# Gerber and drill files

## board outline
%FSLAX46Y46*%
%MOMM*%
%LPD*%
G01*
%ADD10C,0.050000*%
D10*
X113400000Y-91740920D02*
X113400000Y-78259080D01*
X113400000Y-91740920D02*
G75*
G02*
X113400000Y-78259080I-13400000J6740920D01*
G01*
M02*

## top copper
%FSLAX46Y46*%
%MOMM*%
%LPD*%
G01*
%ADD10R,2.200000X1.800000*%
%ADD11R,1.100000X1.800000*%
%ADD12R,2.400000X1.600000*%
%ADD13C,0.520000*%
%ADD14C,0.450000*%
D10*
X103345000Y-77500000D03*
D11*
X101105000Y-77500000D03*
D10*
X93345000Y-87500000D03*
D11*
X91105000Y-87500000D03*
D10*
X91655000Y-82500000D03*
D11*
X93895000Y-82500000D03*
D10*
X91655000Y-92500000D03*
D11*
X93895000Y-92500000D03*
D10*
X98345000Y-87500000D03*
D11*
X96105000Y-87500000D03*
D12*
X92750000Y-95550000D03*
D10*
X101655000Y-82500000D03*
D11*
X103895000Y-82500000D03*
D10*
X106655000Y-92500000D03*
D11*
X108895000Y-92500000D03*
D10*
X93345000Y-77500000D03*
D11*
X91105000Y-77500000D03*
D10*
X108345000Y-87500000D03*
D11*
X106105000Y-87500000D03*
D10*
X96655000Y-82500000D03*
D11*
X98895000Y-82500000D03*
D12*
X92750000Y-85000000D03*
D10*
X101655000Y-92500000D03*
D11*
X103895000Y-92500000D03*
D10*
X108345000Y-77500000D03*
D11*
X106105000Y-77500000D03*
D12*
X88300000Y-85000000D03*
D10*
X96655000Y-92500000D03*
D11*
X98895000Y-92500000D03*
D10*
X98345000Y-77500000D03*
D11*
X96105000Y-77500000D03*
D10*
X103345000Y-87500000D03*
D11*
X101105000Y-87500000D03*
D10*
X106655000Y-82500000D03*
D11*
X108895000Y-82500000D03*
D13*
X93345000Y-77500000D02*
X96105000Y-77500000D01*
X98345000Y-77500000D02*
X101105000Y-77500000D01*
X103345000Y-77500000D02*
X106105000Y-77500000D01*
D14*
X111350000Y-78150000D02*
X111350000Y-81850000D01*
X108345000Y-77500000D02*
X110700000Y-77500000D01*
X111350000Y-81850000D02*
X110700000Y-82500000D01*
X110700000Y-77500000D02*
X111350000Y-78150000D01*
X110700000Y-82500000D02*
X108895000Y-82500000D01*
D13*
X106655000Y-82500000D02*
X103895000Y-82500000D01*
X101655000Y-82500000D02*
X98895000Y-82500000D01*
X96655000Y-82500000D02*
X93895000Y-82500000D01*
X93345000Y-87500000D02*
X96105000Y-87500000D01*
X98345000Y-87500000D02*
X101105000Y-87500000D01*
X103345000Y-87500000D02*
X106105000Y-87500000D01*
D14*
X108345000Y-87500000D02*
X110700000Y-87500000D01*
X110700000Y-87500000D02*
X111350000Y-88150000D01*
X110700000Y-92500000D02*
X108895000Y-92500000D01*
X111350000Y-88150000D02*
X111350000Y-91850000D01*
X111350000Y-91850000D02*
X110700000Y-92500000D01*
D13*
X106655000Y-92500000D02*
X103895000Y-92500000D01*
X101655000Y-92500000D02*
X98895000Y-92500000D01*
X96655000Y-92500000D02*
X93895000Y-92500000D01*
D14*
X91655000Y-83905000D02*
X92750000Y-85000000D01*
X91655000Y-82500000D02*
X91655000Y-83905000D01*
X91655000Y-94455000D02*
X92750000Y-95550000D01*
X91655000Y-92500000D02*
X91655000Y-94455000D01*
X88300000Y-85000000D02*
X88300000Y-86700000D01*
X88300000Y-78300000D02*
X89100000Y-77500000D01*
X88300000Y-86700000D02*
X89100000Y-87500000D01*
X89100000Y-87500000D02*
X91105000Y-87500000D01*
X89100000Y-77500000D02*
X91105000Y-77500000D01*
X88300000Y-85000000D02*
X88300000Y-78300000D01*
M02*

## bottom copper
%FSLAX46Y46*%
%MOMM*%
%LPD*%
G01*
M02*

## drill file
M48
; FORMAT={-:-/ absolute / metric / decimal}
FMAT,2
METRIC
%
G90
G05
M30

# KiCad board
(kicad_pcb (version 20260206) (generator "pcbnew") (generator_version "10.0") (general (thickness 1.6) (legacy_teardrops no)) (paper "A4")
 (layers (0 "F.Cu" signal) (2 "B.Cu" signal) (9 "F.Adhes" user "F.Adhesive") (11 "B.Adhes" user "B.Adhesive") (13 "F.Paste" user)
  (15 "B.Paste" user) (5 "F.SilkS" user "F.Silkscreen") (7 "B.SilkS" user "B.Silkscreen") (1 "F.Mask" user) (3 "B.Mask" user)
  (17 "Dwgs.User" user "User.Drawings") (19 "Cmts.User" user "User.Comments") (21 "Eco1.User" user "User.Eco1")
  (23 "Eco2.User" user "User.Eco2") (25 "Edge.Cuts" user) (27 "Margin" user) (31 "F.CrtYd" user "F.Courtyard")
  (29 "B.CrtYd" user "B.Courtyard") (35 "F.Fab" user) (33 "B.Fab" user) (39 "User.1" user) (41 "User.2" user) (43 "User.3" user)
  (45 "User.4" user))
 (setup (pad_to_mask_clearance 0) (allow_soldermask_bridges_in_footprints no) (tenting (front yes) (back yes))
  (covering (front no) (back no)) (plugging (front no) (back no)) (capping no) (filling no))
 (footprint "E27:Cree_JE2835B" (layer "F.Cu") (at 102.5 77.5 180)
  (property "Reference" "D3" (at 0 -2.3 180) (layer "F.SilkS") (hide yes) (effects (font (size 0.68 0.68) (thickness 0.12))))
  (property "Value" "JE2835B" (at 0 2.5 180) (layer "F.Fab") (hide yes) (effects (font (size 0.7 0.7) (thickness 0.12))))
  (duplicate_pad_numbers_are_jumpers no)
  (pad "1" smd rect (at -0.845 0 180) (size 2.2 1.8) (layers "F.Cu" "F.Mask" "F.Paste") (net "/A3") (solder_paste_margin_ratio -0.2))
  (pad "2" smd rect (at 1.395 0 180) (size 1.1 1.8) (layers "F.Cu" "F.Mask" "F.Paste") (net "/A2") (solder_paste_margin_ratio -0.2)))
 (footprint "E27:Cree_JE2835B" (layer "F.Cu") (at 92.5 87.5 180)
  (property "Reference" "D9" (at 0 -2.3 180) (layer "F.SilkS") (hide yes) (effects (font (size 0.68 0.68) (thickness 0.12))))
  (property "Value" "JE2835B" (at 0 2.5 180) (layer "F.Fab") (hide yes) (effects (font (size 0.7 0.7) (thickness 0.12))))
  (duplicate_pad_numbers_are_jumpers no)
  (pad "1" smd rect (at -0.845 0 180) (size 2.2 1.8) (layers "F.Cu" "F.Mask" "F.Paste") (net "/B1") (solder_paste_margin_ratio -0.2))
  (pad "2" smd rect (at 1.395 0 180) (size 1.1 1.8) (layers "F.Cu" "F.Mask" "F.Paste") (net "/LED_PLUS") (solder_paste_margin_ratio -0.2)))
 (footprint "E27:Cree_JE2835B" (layer "F.Cu") (at 92.5 82.5)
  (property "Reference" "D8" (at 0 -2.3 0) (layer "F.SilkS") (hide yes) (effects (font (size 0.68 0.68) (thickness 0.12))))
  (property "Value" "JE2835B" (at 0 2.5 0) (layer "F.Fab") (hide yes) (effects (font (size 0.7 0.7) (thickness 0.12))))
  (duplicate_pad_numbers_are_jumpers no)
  (pad "1" smd rect (at -0.845 0) (size 2.2 1.8) (layers "F.Cu" "F.Mask" "F.Paste") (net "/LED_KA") (solder_paste_margin_ratio -0.2))
  (pad "2" smd rect (at 1.395 0) (size 1.1 1.8) (layers "F.Cu" "F.Mask" "F.Paste") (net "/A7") (solder_paste_margin_ratio -0.2)))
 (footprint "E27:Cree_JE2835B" (layer "F.Cu") (at 92.5 92.5)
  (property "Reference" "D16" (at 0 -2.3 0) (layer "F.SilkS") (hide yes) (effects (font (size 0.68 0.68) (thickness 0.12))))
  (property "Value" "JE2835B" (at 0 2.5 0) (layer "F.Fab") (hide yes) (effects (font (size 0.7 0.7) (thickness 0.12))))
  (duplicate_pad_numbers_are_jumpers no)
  (pad "1" smd rect (at -0.845 0) (size 2.2 1.8) (layers "F.Cu" "F.Mask" "F.Paste") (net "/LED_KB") (solder_paste_margin_ratio -0.2))
  (pad "2" smd rect (at 1.395 0) (size 1.1 1.8) (layers "F.Cu" "F.Mask" "F.Paste") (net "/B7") (solder_paste_margin_ratio -0.2)))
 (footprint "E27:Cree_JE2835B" (layer "F.Cu") (at 97.5 87.5 180)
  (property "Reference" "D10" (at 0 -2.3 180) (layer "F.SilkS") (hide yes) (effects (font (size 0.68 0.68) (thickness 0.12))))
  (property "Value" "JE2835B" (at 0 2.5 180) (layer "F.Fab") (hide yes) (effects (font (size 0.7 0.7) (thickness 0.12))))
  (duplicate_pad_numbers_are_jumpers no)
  (pad "1" smd rect (at -0.845 0 180) (size 2.2 1.8) (layers "F.Cu" "F.Mask" "F.Paste") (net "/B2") (solder_paste_margin_ratio -0.2))
  (pad "2" smd rect (at 1.395 0 180) (size 1.1 1.8) (layers "F.Cu" "F.Mask" "F.Paste") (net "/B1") (solder_paste_margin_ratio -0.2)))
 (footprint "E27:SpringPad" (layer "F.Cu") (at 92.75 95.55)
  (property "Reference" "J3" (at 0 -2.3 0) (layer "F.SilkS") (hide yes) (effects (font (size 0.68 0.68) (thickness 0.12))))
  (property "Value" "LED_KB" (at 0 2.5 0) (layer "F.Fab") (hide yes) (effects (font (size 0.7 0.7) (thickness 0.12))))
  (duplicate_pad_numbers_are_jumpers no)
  (pad "1" smd rect (at 0 0) (size 2.4 1.6) (layers "F.Cu" "F.Mask") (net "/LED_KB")))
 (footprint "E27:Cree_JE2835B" (layer "F.Cu") (at 102.5 82.5)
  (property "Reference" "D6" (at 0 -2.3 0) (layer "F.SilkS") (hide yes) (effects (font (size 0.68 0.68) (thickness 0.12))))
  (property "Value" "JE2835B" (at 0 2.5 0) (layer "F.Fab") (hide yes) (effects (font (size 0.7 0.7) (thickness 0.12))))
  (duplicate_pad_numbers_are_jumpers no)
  (pad "1" smd rect (at -0.845 0) (size 2.2 1.8) (layers "F.Cu" "F.Mask" "F.Paste") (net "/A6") (solder_paste_margin_ratio -0.2))
  (pad "2" smd rect (at 1.395 0) (size 1.1 1.8) (layers "F.Cu" "F.Mask" "F.Paste") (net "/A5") (solder_paste_margin_ratio -0.2)))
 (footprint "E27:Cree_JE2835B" (layer "F.Cu") (at 107.5 92.5)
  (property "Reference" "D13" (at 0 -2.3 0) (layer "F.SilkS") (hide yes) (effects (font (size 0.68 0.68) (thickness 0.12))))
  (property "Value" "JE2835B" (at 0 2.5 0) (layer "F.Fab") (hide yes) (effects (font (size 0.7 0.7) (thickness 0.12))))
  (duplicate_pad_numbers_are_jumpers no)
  (pad "1" smd rect (at -0.845 0) (size 2.2 1.8) (layers "F.Cu" "F.Mask" "F.Paste") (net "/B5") (solder_paste_margin_ratio -0.2))
  (pad "2" smd rect (at 1.395 0) (size 1.1 1.8) (layers "F.Cu" "F.Mask" "F.Paste") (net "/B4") (solder_paste_margin_ratio -0.2)))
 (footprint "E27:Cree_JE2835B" (layer "F.Cu") (at 92.5 77.5 180)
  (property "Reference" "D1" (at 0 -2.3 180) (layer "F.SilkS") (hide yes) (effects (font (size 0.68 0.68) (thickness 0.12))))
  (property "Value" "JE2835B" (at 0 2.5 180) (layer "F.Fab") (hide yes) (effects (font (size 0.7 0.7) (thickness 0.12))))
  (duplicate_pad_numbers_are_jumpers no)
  (pad "1" smd rect (at -0.845 0 180) (size 2.2 1.8) (layers "F.Cu" "F.Mask" "F.Paste") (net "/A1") (solder_paste_margin_ratio -0.2))
  (pad "2" smd rect (at 1.395 0 180) (size 1.1 1.8) (layers "F.Cu" "F.Mask" "F.Paste") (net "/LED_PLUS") (solder_paste_margin_ratio -0.2)))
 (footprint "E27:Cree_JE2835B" (layer "F.Cu") (at 107.5 87.5 180)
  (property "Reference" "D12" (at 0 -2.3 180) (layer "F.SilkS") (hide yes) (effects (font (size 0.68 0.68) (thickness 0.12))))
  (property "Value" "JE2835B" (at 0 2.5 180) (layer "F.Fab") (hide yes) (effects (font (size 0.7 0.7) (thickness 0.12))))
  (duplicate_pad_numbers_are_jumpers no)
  (pad "1" smd rect (at -0.845 0 180) (size 2.2 1.8) (layers "F.Cu" "F.Mask" "F.Paste") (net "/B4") (solder_paste_margin_ratio -0.2))
  (pad "2" smd rect (at 1.395 0 180) (size 1.1 1.8) (layers "F.Cu" "F.Mask" "F.Paste") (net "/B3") (solder_paste_margin_ratio -0.2)))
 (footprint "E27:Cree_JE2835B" (layer "F.Cu") (at 97.5 82.5)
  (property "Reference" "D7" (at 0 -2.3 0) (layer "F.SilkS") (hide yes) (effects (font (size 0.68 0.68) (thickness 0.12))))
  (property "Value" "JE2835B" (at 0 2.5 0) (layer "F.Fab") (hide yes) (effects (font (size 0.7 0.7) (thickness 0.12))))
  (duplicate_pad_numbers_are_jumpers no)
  (pad "1" smd rect (at -0.845 0) (size 2.2 1.8) (layers "F.Cu" "F.Mask" "F.Paste") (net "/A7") (solder_paste_margin_ratio -0.2))
  (pad "2" smd rect (at 1.395 0) (size 1.1 1.8) (layers "F.Cu" "F.Mask" "F.Paste") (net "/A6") (solder_paste_margin_ratio -0.2)))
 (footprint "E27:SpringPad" (layer "F.Cu") (at 92.75 85)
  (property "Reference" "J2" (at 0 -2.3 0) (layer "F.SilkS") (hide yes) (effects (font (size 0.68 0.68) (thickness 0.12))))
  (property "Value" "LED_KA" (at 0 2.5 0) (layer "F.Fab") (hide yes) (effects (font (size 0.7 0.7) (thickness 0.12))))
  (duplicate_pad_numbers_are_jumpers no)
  (pad "1" smd rect (at 0 0) (size 2.4 1.6) (layers "F.Cu" "F.Mask") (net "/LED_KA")))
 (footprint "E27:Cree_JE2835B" (layer "F.Cu") (at 102.5 92.5)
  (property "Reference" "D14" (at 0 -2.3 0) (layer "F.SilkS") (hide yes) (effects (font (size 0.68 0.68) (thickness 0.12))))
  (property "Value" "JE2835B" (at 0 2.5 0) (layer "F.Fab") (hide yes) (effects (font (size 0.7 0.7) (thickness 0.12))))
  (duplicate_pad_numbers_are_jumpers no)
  (pad "1" smd rect (at -0.845 0) (size 2.2 1.8) (layers "F.Cu" "F.Mask" "F.Paste") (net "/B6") (solder_paste_margin_ratio -0.2))
  (pad "2" smd rect (at 1.395 0) (size 1.1 1.8) (layers "F.Cu" "F.Mask" "F.Paste") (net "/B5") (solder_paste_margin_ratio -0.2)))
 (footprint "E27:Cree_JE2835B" (layer "F.Cu") (at 107.5 77.5 180)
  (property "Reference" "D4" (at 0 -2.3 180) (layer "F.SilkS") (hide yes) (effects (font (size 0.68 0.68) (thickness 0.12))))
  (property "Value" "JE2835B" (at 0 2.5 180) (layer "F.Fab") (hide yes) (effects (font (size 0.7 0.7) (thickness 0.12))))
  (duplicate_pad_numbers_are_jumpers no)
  (pad "1" smd rect (at -0.845 0 180) (size 2.2 1.8) (layers "F.Cu" "F.Mask" "F.Paste") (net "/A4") (solder_paste_margin_ratio -0.2))
  (pad "2" smd rect (at 1.395 0 180) (size 1.1 1.8) (layers "F.Cu" "F.Mask" "F.Paste") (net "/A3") (solder_paste_margin_ratio -0.2)))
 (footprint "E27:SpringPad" (layer "F.Cu") (at 88.3 85)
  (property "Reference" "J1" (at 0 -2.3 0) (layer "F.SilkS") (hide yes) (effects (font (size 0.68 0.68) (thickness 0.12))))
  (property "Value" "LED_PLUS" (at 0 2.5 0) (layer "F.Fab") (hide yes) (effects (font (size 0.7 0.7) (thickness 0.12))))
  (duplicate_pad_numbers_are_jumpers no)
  (pad "1" smd rect (at 0 0) (size 2.4 1.6) (layers "F.Cu" "F.Mask") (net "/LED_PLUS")))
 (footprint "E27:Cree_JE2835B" (layer "F.Cu") (at 97.5 92.5)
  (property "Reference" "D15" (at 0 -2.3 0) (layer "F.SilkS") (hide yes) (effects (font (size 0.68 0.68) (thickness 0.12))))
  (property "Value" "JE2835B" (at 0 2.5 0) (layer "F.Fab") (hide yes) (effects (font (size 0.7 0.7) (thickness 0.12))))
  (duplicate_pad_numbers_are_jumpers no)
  (pad "1" smd rect (at -0.845 0) (size 2.2 1.8) (layers "F.Cu" "F.Mask" "F.Paste") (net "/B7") (solder_paste_margin_ratio -0.2))
  (pad "2" smd rect (at 1.395 0) (size 1.1 1.8) (layers "F.Cu" "F.Mask" "F.Paste") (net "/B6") (solder_paste_margin_ratio -0.2)))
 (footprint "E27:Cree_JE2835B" (layer "F.Cu") (at 97.5 77.5 180)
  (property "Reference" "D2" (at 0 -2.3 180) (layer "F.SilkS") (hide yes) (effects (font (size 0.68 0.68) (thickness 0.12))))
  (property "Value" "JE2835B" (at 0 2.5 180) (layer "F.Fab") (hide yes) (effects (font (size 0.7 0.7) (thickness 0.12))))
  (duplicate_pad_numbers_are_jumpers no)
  (pad "1" smd rect (at -0.845 0 180) (size 2.2 1.8) (layers "F.Cu" "F.Mask" "F.Paste") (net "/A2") (solder_paste_margin_ratio -0.2))
  (pad "2" smd rect (at 1.395 0 180) (size 1.1 1.8) (layers "F.Cu" "F.Mask" "F.Paste") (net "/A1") (solder_paste_margin_ratio -0.2)))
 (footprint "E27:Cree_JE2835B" (layer "F.Cu") (at 102.5 87.5 180)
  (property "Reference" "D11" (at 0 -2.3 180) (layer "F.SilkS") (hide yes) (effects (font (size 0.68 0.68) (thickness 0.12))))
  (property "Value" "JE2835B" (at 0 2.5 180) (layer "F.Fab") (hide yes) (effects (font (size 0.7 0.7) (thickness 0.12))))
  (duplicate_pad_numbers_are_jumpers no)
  (pad "1" smd rect (at -0.845 0 180) (size 2.2 1.8) (layers "F.Cu" "F.Mask" "F.Paste") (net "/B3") (solder_paste_margin_ratio -0.2))
  (pad "2" smd rect (at 1.395 0 180) (size 1.1 1.8) (layers "F.Cu" "F.Mask" "F.Paste") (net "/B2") (solder_paste_margin_ratio -0.2)))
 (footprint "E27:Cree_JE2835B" (layer "F.Cu") (at 107.5 82.5)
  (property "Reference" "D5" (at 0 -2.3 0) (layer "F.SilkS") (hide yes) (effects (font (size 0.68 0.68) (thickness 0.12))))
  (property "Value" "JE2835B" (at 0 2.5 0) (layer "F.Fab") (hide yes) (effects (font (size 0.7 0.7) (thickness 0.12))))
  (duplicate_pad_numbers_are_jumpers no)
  (pad "1" smd rect (at -0.845 0) (size 2.2 1.8) (layers "F.Cu" "F.Mask" "F.Paste") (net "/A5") (solder_paste_margin_ratio -0.2))
  (pad "2" smd rect (at 1.395 0) (size 1.1 1.8) (layers "F.Cu" "F.Mask" "F.Paste") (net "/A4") (solder_paste_margin_ratio -0.2)))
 (gr_line (start 113.4 91.74092) (end 113.4 78.25908) (stroke (width 0.05) (type default)) (layer "Edge.Cuts"))
 (gr_arc (start 113.4 91.74092) (mid 85 85) (end 113.4 78.25908) (stroke (width 0.05) (type default)) (layer "Edge.Cuts"))
 (segment (start 93.345 77.5) (end 96.105 77.5) (width 0.52) (layer "F.Cu") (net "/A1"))
 (segment (start 98.345 77.5) (end 101.105 77.5) (width 0.52) (layer "F.Cu") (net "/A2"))
 (segment (start 103.345 77.5) (end 106.105 77.5) (width 0.52) (layer "F.Cu") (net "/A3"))
 (segment (start 111.35 78.15) (end 111.35 81.85) (width 0.45) (layer "F.Cu") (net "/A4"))
 (segment (start 108.345 77.5) (end 110.7 77.5) (width 0.45) (layer "F.Cu") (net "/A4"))
 (segment (start 111.35 81.85) (end 110.7 82.5) (width 0.45) (layer "F.Cu") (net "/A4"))
 (segment (start 110.7 77.5) (end 111.35 78.15) (width 0.45) (layer "F.Cu") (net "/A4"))
 (segment (start 110.7 82.5) (end 108.895 82.5) (width 0.45) (layer "F.Cu") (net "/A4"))
 (segment (start 106.655 82.5) (end 103.895 82.5) (width 0.52) (layer "F.Cu") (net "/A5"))
 (segment (start 101.655 82.5) (end 98.895 82.5) (width 0.52) (layer "F.Cu") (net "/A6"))
 (segment (start 96.655 82.5) (end 93.895 82.5) (width 0.52) (layer "F.Cu") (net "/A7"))
 (segment (start 93.345 87.5) (end 96.105 87.5) (width 0.52) (layer "F.Cu") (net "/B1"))
 (segment (start 98.345 87.5) (end 101.105 87.5) (width 0.52) (layer "F.Cu") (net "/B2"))
 (segment (start 103.345 87.5) (end 106.105 87.5) (width 0.52) (layer "F.Cu") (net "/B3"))
 (segment (start 108.345 87.5) (end 110.7 87.5) (width 0.45) (layer "F.Cu") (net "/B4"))
 (segment (start 110.7 87.5) (end 111.35 88.15) (width 0.45) (layer "F.Cu") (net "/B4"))
 (segment (start 110.7 92.5) (end 108.895 92.5) (width 0.45) (layer "F.Cu") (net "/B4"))
 (segment (start 111.35 88.15) (end 111.35 91.85) (width 0.45) (layer "F.Cu") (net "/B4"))
 (segment (start 111.35 91.85) (end 110.7 92.5) (width 0.45) (layer "F.Cu") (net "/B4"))
 (segment (start 106.655 92.5) (end 103.895 92.5) (width 0.52) (layer "F.Cu") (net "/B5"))
 (segment (start 101.655 92.5) (end 98.895 92.5) (width 0.52) (layer "F.Cu") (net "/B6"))
 (segment (start 96.655 92.5) (end 93.895 92.5) (width 0.52) (layer "F.Cu") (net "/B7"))
 (segment (start 91.655 83.905) (end 92.75 85) (width 0.45) (layer "F.Cu") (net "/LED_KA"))
 (segment (start 91.655 82.5) (end 91.655 83.905) (width 0.45) (layer "F.Cu") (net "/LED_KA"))
 (segment (start 91.655 94.455) (end 92.75 95.55) (width 0.45) (layer "F.Cu") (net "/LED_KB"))
 (segment (start 91.655 92.5) (end 91.655 94.455) (width 0.45) (layer "F.Cu") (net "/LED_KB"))
 (segment (start 88.3 85) (end 88.3 86.7) (width 0.45) (layer "F.Cu") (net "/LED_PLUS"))
 (segment (start 88.3 78.3) (end 89.1 77.5) (width 0.45) (layer "F.Cu") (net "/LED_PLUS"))
 (segment (start 88.3 86.7) (end 89.1 87.5) (width 0.45) (layer "F.Cu") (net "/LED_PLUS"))
 (segment (start 89.1 87.5) (end 91.105 87.5) (width 0.45) (layer "F.Cu") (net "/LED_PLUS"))
 (segment (start 89.1 77.5) (end 91.105 77.5) (width 0.45) (layer "F.Cu") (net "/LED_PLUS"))
 (segment (start 88.3 85) (end 88.3 78.3) (width 0.45) (layer "F.Cu") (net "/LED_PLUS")))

